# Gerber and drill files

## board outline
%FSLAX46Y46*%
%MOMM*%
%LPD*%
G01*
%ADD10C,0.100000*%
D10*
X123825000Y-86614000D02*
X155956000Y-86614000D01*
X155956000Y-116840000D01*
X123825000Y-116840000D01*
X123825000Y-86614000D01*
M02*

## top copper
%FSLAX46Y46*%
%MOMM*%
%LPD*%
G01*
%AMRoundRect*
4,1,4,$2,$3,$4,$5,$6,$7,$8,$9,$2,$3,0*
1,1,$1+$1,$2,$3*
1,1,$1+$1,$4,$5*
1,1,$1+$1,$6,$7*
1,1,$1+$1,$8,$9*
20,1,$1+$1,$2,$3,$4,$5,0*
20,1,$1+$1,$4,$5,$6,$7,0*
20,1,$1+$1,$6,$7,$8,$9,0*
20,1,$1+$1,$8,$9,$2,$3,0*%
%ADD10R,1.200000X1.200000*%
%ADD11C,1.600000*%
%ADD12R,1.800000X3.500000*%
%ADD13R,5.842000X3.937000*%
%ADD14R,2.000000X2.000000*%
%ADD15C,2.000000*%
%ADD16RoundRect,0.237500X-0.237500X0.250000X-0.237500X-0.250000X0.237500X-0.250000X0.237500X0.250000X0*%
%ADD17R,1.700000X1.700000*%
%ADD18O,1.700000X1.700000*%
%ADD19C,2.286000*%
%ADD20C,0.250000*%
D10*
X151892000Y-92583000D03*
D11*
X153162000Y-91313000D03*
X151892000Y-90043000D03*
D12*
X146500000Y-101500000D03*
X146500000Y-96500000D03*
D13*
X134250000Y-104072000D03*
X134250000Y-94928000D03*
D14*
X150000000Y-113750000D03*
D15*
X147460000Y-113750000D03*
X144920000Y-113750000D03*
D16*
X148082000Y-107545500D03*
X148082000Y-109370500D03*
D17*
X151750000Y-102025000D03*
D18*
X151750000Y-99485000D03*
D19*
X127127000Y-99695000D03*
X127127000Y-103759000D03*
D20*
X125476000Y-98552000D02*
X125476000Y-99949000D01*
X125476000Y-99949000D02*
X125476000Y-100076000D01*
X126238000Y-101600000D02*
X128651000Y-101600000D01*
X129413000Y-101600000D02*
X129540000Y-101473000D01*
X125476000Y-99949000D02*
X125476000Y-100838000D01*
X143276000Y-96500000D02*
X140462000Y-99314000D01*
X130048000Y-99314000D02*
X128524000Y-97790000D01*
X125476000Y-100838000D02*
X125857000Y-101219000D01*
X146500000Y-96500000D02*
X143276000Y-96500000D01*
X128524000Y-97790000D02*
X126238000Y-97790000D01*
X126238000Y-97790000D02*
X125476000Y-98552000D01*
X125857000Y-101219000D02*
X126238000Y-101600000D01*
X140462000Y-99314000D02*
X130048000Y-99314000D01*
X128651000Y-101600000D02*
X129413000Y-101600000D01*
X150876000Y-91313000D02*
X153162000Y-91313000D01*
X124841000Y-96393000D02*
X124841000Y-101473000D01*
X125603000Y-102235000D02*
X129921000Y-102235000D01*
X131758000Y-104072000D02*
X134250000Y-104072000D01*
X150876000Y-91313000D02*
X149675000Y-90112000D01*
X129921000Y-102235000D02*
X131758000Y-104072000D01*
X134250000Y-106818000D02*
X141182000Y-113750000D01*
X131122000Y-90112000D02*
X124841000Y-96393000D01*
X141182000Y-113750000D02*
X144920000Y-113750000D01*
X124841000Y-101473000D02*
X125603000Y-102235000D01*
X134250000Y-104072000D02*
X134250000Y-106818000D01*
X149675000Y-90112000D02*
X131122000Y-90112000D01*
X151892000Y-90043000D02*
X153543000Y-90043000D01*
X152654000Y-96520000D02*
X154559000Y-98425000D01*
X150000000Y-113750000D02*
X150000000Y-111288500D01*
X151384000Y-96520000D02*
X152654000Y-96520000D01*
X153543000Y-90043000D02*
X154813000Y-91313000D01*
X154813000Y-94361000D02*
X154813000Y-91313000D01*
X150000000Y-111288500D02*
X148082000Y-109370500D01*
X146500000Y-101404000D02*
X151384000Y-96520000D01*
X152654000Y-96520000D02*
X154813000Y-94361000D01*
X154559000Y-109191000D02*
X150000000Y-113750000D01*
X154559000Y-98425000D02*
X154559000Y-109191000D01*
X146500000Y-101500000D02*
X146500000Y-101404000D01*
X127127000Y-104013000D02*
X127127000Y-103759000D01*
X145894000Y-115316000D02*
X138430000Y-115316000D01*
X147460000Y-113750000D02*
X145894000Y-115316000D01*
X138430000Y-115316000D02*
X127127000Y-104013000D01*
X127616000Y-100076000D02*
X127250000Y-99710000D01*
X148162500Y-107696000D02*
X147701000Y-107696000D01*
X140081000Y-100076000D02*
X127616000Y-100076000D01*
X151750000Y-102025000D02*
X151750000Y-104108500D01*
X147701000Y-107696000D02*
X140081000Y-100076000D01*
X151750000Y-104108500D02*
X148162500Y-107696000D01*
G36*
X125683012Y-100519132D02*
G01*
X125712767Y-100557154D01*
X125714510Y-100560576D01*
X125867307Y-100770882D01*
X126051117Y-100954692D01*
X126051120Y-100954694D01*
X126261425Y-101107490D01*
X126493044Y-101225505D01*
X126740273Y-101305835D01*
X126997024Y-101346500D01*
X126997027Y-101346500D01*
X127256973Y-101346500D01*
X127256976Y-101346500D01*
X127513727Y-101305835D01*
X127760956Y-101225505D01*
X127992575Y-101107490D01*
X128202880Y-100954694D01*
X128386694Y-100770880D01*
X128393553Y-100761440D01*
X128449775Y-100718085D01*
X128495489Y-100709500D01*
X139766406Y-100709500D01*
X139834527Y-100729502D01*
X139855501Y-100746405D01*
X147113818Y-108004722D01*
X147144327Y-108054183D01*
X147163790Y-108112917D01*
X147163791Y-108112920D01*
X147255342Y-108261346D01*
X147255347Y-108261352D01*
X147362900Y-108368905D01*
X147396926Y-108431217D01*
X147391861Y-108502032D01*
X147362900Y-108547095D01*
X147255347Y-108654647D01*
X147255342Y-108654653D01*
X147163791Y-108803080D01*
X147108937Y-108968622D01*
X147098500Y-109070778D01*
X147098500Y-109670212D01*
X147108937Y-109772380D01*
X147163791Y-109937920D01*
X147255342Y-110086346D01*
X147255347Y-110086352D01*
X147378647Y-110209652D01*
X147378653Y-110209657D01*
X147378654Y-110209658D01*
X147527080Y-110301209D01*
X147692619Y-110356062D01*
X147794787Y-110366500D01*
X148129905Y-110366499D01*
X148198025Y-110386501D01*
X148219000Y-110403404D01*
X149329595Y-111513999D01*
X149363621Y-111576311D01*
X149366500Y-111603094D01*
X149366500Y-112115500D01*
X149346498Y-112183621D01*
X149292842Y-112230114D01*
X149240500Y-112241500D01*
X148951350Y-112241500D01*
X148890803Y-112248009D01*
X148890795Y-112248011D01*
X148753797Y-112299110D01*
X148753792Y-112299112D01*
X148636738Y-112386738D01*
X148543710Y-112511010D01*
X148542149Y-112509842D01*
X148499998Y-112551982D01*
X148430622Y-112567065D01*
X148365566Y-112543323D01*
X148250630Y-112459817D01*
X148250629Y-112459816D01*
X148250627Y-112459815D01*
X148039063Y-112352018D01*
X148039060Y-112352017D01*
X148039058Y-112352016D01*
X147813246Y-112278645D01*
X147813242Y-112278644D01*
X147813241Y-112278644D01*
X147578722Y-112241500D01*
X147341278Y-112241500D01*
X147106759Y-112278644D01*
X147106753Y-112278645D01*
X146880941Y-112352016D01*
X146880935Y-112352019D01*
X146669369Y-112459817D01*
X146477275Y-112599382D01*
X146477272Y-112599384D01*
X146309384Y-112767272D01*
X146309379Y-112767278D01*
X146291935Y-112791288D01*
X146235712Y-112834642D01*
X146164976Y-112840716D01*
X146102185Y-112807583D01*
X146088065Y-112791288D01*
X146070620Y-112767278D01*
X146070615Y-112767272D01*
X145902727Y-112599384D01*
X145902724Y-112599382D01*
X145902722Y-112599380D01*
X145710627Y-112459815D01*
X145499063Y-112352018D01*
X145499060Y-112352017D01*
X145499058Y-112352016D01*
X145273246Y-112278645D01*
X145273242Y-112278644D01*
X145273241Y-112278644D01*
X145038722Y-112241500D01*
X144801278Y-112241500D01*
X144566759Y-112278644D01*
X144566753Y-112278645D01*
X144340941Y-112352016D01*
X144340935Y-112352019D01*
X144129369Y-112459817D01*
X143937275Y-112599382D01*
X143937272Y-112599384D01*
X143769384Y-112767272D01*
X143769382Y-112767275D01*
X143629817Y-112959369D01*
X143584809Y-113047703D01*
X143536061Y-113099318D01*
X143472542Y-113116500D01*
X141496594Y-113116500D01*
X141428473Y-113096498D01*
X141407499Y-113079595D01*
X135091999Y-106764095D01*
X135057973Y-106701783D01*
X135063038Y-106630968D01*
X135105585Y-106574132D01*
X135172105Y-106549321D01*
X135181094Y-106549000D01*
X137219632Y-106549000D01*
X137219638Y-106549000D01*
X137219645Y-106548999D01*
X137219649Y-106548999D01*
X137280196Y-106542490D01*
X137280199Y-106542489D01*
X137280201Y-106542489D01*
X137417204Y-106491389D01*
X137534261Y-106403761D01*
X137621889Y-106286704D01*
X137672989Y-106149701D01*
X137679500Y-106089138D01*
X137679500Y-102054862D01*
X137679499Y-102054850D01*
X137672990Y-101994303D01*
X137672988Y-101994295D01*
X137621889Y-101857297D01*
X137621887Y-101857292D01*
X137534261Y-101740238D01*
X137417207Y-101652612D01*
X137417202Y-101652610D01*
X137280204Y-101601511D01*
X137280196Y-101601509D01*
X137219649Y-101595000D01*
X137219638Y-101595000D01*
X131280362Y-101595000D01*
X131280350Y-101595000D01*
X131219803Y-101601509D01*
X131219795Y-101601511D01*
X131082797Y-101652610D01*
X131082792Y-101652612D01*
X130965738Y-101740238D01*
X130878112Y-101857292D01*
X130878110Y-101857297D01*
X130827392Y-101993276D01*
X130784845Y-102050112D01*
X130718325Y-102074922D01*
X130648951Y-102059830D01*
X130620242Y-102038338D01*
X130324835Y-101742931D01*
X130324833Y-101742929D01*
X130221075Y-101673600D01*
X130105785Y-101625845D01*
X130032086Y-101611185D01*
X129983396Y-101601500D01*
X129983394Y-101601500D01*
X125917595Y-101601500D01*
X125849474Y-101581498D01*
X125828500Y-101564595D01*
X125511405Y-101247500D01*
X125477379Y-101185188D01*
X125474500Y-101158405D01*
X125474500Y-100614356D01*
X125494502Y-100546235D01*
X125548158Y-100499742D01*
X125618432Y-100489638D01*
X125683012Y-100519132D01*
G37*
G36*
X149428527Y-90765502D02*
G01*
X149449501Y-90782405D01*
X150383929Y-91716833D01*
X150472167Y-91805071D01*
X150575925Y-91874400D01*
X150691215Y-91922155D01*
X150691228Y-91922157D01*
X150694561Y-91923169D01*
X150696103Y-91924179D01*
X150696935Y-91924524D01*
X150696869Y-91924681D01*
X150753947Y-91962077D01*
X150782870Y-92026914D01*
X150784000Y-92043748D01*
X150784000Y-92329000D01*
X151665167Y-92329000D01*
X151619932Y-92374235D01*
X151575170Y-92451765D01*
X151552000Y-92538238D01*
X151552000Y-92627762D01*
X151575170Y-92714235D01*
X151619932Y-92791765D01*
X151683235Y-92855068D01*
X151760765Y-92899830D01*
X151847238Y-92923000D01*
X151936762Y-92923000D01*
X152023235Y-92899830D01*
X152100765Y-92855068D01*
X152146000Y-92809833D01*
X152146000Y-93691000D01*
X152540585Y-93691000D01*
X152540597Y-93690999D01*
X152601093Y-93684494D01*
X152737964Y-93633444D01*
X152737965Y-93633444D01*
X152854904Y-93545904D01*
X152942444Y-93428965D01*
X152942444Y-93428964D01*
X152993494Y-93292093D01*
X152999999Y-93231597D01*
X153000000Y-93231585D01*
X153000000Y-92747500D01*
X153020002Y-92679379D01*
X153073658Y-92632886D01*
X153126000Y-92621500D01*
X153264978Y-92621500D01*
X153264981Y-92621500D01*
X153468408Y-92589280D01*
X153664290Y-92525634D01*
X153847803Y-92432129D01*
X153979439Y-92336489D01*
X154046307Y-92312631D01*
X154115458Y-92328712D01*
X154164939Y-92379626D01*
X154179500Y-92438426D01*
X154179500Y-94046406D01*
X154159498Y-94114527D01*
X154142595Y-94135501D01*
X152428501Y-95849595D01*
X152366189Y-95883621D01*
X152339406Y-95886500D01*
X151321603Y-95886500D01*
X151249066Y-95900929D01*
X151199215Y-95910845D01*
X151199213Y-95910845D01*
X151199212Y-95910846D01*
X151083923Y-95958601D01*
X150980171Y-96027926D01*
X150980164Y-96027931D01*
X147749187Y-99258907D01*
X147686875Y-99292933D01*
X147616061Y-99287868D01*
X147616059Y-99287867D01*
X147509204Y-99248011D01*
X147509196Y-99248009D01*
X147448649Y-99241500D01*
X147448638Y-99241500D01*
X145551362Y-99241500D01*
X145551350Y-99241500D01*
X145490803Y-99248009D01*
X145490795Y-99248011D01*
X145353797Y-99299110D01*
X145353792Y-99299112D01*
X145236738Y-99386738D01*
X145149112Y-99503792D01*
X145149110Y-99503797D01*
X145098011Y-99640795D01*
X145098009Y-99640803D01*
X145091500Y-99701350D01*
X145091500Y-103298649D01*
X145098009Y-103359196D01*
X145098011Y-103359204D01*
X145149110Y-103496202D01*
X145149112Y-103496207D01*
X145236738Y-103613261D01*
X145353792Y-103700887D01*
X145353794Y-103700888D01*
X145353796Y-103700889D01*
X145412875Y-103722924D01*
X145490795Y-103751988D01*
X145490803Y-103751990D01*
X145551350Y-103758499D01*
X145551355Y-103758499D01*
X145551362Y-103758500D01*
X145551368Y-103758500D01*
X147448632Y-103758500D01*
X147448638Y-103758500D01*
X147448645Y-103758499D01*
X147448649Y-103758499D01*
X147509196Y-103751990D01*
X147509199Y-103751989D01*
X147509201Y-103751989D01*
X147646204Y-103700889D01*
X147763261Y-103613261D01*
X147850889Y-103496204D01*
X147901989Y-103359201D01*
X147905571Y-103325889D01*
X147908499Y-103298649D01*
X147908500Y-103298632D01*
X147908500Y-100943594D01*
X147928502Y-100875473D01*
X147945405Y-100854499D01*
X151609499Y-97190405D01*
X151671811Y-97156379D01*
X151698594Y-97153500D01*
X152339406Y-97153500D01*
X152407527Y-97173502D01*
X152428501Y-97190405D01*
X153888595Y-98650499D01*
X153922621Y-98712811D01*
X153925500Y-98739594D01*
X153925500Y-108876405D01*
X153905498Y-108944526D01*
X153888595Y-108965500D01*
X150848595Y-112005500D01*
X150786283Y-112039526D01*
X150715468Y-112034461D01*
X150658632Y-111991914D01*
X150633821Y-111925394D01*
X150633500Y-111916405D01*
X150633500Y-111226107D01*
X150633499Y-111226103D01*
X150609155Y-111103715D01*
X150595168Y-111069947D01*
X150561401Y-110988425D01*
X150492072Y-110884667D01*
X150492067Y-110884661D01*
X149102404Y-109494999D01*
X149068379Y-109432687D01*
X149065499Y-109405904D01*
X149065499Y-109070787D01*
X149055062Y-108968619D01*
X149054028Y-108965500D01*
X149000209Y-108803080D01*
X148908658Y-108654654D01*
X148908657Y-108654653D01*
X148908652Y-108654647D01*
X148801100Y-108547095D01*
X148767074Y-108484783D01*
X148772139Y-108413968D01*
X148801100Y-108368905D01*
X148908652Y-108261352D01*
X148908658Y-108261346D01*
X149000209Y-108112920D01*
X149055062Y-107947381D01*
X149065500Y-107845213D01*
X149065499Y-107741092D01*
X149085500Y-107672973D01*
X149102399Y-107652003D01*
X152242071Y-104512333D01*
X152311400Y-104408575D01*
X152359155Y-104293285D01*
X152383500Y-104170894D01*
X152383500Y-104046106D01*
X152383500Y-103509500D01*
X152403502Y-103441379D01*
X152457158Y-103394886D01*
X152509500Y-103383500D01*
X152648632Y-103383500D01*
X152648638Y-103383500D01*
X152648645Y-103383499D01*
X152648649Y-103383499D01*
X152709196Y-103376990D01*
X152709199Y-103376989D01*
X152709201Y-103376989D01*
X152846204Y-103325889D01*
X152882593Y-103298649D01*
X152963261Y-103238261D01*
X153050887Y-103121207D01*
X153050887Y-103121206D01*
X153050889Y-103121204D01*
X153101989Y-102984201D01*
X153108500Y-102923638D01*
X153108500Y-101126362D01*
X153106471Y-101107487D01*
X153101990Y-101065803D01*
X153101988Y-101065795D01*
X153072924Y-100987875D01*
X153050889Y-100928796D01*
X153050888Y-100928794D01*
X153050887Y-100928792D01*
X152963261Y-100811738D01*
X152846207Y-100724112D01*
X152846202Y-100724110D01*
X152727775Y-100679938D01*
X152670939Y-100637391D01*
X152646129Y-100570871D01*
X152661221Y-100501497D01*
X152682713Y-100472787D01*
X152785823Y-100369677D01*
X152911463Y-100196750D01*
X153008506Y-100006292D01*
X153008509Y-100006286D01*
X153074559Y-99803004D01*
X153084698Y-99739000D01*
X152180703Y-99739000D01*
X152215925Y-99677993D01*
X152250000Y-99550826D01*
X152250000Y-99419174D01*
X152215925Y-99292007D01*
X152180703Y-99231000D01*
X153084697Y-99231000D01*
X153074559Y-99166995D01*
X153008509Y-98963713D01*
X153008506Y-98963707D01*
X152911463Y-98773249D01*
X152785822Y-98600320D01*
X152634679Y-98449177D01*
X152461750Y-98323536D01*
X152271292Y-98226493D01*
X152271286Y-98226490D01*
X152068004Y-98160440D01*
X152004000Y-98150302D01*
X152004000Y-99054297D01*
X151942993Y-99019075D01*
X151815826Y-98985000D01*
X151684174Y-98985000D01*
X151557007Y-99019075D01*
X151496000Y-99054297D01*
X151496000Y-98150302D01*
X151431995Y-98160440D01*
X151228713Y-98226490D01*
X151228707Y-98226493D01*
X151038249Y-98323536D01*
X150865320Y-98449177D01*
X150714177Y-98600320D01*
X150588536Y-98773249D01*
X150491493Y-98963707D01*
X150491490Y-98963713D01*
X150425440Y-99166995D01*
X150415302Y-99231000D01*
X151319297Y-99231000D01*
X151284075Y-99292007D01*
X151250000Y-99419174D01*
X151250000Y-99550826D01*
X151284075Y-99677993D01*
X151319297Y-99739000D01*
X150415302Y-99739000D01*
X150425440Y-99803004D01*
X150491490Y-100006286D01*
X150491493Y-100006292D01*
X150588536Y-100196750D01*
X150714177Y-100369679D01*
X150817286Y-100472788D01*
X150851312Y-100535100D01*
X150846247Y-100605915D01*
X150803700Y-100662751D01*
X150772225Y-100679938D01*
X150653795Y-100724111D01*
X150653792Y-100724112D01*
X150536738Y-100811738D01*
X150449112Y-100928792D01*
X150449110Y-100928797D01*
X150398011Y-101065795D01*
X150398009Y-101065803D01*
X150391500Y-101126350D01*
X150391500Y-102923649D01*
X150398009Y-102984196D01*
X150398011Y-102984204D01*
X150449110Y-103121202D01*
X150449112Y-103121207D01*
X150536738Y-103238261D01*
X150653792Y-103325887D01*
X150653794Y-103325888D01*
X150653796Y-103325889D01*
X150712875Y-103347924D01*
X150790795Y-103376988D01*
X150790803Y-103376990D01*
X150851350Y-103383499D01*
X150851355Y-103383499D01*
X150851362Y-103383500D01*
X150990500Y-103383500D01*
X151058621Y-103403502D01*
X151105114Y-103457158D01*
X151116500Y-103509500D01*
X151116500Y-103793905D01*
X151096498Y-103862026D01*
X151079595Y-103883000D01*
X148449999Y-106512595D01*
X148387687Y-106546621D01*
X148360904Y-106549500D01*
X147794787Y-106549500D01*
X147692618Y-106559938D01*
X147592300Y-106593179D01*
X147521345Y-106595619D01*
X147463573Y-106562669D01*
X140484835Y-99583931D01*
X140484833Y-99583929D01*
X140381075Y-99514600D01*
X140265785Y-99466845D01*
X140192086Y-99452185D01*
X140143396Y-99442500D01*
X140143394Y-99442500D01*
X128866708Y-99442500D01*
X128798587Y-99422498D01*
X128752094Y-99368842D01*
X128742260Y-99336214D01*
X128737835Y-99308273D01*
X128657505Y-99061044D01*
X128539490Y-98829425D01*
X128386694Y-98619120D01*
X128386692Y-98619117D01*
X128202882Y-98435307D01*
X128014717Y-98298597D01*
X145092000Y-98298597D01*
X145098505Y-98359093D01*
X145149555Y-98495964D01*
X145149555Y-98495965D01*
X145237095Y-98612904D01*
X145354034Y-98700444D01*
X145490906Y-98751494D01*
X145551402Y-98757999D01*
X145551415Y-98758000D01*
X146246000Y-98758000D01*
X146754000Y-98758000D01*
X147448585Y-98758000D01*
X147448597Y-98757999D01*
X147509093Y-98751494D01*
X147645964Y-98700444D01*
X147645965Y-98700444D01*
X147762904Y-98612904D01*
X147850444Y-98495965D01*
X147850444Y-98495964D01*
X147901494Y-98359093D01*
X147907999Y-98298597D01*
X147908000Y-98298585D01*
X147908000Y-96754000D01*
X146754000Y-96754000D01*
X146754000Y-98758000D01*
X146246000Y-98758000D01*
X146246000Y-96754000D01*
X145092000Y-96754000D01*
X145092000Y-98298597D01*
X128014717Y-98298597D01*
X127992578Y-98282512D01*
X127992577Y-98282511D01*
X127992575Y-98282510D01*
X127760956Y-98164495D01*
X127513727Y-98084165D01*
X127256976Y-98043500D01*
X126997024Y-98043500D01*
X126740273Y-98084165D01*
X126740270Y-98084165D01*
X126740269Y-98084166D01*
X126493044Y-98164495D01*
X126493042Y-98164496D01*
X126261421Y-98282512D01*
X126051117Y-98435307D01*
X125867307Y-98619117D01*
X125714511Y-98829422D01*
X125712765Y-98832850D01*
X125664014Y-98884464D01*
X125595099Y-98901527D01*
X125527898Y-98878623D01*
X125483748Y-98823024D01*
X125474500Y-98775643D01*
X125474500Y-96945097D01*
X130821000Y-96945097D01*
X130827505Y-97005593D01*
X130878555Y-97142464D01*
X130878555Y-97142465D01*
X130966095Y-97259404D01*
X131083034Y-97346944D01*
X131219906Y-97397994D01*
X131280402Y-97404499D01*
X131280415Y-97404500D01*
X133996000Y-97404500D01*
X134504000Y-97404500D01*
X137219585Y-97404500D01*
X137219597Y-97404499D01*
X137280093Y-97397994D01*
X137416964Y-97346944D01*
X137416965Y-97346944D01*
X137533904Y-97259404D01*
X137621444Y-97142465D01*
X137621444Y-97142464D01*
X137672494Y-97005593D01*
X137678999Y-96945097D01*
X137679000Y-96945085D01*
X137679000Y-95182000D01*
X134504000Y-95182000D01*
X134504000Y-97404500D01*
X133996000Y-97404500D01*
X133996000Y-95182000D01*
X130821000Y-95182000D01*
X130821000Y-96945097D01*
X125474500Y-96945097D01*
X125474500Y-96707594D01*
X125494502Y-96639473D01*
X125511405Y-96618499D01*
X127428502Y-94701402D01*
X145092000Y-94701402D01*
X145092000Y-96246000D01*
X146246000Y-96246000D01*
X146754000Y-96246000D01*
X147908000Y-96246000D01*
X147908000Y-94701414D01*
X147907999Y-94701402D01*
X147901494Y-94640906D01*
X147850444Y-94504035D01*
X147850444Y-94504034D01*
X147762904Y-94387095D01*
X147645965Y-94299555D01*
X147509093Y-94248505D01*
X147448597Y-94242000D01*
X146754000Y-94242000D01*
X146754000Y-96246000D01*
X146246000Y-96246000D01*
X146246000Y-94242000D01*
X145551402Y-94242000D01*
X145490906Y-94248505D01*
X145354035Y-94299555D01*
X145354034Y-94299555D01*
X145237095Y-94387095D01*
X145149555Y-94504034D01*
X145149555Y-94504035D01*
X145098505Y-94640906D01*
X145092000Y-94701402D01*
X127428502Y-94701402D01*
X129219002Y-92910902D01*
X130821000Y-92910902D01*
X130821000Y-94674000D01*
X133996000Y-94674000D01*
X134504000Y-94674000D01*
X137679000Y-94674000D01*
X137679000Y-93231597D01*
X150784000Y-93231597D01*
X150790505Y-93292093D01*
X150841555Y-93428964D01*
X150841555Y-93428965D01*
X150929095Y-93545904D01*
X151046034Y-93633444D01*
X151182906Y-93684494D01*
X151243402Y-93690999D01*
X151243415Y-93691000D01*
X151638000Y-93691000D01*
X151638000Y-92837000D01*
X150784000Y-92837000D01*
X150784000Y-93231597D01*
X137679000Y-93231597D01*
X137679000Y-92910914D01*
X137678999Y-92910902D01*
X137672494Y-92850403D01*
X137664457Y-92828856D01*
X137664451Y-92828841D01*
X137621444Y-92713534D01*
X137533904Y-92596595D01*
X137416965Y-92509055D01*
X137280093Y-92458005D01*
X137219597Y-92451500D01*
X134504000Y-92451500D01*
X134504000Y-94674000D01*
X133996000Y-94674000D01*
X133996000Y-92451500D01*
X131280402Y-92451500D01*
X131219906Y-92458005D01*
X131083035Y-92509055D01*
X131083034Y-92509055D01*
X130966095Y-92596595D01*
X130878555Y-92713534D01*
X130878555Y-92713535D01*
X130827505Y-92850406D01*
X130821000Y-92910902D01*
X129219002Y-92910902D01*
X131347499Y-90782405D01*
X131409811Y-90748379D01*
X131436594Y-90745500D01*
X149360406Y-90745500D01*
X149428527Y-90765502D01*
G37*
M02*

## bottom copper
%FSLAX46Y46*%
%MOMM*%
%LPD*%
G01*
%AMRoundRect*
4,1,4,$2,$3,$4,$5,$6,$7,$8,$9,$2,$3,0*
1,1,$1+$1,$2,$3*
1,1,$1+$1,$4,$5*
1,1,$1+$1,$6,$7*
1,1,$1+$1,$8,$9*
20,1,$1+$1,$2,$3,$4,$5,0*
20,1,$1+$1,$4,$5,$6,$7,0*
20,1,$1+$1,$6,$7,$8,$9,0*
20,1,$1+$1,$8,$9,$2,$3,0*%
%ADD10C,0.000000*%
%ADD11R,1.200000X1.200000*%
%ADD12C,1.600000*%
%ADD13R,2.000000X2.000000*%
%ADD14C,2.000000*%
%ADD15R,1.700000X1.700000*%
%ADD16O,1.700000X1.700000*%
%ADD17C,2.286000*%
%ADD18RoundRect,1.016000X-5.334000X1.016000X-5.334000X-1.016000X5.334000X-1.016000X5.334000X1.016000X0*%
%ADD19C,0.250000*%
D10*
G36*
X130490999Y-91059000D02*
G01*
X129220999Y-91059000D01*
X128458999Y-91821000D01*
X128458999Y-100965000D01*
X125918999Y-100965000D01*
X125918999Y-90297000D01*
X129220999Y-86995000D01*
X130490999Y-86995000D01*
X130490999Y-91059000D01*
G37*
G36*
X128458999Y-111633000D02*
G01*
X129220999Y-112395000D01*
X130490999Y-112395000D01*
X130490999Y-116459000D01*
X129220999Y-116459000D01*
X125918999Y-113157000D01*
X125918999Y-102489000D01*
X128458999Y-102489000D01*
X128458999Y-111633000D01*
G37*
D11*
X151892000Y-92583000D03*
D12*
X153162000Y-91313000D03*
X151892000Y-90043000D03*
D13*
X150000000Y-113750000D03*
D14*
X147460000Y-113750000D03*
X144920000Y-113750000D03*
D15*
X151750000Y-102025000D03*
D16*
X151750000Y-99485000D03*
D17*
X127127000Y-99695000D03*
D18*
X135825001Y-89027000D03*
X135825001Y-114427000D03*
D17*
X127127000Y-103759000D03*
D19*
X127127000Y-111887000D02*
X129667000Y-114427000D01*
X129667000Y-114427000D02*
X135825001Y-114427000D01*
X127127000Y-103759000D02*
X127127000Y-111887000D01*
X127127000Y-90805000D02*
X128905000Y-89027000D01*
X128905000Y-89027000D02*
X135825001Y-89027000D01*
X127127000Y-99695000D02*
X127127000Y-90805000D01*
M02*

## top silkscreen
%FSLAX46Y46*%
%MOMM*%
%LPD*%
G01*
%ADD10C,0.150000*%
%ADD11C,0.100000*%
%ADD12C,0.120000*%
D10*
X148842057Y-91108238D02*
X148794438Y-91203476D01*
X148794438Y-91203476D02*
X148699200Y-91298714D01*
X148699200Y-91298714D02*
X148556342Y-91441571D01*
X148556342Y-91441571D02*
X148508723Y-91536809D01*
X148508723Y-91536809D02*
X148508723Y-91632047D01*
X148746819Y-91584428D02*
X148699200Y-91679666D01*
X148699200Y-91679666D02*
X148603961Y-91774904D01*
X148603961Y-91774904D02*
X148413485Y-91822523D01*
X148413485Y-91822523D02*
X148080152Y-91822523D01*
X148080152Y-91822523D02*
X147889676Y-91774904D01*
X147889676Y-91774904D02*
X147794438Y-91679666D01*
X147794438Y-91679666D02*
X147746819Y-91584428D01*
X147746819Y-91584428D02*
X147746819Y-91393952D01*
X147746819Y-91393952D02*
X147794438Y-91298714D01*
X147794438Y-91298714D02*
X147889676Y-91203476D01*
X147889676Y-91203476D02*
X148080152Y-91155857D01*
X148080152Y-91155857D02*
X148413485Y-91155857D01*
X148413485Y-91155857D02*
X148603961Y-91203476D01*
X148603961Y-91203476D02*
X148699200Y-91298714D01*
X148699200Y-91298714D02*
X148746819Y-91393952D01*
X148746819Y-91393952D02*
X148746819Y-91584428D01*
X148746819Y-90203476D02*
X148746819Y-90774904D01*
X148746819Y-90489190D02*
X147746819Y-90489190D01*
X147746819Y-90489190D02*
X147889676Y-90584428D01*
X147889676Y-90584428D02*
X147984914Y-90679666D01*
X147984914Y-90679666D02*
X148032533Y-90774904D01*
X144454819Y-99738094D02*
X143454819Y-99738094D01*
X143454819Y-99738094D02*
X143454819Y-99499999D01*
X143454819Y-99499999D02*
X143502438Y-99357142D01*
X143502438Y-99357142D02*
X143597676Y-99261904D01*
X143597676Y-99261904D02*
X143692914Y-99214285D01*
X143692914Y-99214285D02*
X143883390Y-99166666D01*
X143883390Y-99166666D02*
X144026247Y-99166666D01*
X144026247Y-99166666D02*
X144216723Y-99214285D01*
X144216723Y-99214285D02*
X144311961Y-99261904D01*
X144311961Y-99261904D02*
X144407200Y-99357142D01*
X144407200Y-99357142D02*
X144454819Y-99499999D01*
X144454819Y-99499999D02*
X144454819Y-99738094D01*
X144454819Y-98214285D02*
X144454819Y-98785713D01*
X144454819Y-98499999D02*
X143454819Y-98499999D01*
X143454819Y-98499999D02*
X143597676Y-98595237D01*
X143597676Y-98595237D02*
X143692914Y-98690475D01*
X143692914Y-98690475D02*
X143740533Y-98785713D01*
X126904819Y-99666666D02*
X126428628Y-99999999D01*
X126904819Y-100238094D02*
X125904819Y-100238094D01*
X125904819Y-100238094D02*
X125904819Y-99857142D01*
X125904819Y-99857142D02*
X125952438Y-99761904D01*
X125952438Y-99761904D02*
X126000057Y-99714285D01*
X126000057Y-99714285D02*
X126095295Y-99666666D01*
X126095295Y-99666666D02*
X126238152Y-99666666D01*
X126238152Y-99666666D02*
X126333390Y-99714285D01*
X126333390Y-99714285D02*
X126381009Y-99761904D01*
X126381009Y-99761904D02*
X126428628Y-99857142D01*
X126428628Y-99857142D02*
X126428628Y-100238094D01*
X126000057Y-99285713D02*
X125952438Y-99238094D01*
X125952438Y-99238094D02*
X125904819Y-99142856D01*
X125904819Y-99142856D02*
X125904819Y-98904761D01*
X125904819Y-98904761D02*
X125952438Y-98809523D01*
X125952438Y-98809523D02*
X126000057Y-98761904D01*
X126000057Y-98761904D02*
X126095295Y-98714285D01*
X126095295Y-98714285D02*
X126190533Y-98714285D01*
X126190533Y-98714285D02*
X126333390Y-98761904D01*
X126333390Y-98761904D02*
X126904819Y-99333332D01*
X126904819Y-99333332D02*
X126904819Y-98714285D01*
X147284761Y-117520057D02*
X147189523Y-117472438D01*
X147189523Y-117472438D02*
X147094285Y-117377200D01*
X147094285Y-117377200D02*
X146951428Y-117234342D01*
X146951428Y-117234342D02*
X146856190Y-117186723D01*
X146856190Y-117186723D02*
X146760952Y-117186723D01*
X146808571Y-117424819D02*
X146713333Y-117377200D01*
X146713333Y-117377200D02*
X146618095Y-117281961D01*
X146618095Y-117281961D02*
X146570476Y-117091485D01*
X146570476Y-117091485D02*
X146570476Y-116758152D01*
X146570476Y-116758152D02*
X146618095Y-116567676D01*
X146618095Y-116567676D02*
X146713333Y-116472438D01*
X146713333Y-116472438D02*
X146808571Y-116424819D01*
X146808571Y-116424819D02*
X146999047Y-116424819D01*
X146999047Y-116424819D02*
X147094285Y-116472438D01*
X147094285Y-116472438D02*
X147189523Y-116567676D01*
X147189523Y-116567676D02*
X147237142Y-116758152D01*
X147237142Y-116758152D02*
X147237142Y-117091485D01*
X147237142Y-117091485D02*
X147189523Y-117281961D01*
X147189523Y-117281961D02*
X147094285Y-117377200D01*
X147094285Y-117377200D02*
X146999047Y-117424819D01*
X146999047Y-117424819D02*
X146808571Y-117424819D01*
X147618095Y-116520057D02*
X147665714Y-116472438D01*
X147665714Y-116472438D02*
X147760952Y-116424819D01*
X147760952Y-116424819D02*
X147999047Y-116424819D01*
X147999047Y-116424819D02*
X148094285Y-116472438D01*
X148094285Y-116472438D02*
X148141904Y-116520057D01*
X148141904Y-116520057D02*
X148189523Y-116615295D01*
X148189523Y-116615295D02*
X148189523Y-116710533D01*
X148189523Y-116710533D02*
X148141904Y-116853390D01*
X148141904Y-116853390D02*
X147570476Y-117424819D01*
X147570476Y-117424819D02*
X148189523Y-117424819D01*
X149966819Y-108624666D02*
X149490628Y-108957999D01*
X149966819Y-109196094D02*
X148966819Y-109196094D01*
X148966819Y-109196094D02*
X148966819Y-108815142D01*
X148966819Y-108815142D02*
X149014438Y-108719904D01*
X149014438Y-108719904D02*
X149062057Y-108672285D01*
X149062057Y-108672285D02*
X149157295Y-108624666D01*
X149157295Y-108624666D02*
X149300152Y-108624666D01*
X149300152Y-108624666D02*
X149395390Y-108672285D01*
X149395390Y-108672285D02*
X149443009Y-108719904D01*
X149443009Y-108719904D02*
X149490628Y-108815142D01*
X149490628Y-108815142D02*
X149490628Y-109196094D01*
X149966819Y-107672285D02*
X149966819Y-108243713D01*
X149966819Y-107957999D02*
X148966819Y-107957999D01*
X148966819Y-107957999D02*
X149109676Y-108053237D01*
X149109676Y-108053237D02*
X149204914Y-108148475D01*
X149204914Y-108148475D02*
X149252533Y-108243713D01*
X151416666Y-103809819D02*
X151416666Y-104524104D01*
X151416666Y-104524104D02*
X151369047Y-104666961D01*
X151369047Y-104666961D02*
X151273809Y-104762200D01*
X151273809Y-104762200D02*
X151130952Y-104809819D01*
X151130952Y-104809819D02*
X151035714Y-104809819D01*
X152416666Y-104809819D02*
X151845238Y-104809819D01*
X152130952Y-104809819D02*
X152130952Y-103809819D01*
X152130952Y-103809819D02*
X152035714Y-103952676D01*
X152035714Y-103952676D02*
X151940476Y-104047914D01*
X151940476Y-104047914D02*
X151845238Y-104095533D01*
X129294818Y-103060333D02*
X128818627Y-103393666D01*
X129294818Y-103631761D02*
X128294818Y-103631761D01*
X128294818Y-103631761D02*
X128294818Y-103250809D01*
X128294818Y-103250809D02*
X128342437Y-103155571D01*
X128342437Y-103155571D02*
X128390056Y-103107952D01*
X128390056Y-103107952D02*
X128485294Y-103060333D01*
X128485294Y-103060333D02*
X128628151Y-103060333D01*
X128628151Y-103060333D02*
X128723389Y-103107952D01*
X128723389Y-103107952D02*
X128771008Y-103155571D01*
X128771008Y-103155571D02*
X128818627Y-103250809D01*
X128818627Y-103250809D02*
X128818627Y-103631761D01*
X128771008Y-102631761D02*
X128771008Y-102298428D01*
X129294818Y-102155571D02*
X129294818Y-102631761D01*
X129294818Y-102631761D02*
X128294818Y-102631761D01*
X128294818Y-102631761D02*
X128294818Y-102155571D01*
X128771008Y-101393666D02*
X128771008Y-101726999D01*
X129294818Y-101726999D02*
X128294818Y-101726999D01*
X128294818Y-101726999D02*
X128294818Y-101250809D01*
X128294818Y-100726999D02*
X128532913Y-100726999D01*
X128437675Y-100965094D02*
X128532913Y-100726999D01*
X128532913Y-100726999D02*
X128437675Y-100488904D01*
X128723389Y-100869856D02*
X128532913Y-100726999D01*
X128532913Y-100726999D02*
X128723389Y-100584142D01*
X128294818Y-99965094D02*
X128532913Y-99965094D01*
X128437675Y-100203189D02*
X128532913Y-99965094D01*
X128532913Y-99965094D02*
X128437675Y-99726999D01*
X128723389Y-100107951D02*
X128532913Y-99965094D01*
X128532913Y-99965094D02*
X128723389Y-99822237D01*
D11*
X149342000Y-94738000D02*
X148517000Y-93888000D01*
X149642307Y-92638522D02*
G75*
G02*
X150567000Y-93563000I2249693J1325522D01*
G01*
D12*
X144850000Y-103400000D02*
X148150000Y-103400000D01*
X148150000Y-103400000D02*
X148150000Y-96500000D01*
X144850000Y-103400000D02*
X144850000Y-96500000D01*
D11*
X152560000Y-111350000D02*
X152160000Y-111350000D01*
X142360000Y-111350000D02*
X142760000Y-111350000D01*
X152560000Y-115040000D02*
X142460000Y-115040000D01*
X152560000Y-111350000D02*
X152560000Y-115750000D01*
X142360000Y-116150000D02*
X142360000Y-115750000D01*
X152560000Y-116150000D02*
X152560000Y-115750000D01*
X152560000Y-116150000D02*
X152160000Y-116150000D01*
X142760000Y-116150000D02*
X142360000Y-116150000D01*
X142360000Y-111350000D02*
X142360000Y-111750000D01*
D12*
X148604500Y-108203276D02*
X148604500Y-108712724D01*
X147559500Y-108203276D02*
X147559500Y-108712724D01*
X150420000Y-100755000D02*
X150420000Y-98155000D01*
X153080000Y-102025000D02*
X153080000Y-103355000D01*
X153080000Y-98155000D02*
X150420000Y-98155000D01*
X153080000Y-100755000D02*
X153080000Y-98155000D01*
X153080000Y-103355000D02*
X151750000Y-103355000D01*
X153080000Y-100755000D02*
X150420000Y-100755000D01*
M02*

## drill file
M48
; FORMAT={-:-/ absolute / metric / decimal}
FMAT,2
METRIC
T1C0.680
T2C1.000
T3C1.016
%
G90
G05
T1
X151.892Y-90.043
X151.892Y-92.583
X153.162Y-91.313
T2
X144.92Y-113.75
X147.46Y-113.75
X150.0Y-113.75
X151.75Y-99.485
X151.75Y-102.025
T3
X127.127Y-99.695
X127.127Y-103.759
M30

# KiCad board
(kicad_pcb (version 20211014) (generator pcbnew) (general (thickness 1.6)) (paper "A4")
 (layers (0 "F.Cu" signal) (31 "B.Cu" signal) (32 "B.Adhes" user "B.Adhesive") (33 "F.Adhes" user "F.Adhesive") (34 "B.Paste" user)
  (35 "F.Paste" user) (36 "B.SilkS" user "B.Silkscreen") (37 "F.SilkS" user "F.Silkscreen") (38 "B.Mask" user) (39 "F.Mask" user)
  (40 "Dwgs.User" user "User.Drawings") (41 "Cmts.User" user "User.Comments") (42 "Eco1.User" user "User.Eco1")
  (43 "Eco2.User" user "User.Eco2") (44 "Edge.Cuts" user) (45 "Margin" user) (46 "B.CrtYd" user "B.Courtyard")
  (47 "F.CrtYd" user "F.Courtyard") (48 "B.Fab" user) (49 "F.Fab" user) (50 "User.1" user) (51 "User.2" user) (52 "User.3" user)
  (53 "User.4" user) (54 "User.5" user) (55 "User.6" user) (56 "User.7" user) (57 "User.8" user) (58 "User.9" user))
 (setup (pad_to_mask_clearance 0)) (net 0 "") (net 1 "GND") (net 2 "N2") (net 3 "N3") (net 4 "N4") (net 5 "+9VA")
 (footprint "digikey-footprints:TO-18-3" (layer "F.Cu") (at 151.892 92.583 90)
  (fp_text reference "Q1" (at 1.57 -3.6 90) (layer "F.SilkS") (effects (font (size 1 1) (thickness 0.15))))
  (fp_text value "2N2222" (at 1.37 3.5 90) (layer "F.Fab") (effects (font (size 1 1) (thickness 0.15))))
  (fp_line (start -2.155 -2.55) (end -1.305 -3.375) (layer "F.SilkS") (width 0.1))
  (fp_arc (start -0.055522 -2.249693) (mid 3.116581 1.846151) (end -0.98 -1.325) (layer "F.SilkS") (width 0.1))
  (pad "1" thru_hole rect locked (at 0 0 90) (size 1.2 1.2) (drill 0.68) (layers *.Cu *.Mask) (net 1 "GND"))
  (pad "2" thru_hole circle locked (at 1.27 1.27 90) (size 1.6 1.6) (drill 0.68) (layers *.Cu *.Mask) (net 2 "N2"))
  (pad "3" thru_hole circle locked (at 2.54 0 90) (size 1.6 1.6) (drill 0.68) (layers *.Cu *.Mask) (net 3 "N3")))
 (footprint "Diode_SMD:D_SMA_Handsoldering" (layer "F.Cu") (at 146.5 99 90)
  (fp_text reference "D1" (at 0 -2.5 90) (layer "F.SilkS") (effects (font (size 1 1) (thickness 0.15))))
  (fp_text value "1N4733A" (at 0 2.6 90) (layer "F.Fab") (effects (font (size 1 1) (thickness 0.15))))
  (fp_line (start -4.4 -1.65) (end -4.4 1.65) (layer "F.SilkS") (width 0.12))
  (fp_line (start -4.4 1.65) (end 2.5 1.65) (layer "F.SilkS") (width 0.12))
  (fp_line (start -4.4 -1.65) (end 2.5 -1.65) (layer "F.SilkS") (width 0.12))
  (pad "1" smd rect locked (at -2.5 0 90) (size 3.5 1.8) (layers "F.Cu" "F.Paste" "F.Mask") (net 3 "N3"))
  (pad "2" smd rect locked (at 2.5 0 90) (size 3.5 1.8) (layers "F.Cu" "F.Paste" "F.Mask") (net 1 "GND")))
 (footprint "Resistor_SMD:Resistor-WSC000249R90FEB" (layer "F.Cu") (at 134.25 99.5 90)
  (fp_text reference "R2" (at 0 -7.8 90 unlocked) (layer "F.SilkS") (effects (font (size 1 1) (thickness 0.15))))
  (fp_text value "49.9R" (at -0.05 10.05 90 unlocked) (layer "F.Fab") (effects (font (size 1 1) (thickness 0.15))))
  (pad "1" smd rect (at -4.572 0 90) (size 3.937 5.842) (layers "F.Cu" "F.Paste" "F.Mask") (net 2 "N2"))
  (pad "2" smd rect (at 4.572 0 90) (size 3.937 5.842) (layers "F.Cu" "F.Paste" "F.Mask") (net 1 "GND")))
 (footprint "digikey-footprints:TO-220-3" (layer "F.Cu") (at 150 113.75 180)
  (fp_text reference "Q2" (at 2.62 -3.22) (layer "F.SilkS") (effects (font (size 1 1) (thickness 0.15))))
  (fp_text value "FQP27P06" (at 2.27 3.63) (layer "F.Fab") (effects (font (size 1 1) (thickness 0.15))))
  (fp_line (start -2.56 2.4) (end -2.16 2.4) (layer "F.SilkS") (width 0.1))
  (fp_line (start 7.64 2.4) (end 7.24 2.4) (layer "F.SilkS") (width 0.1))
  (fp_line (start -2.56 -1.29) (end 7.54 -1.29) (layer "F.SilkS") (width 0.1))
  (fp_line (start -2.56 2.4) (end -2.56 -2) (layer "F.SilkS") (width 0.1))
  (fp_line (start 7.64 -2.4) (end 7.64 -2) (layer "F.SilkS") (width 0.1))
  (fp_line (start -2.56 -2.4) (end -2.56 -2) (layer "F.SilkS") (width 0.1))
  (fp_line (start -2.56 -2.4) (end -2.16 -2.4) (layer "F.SilkS") (width 0.1))
  (fp_line (start 7.24 -2.4) (end 7.64 -2.4) (layer "F.SilkS") (width 0.1))
  (fp_line (start 7.64 2.4) (end 7.64 2) (layer "F.SilkS") (width 0.1))
  (pad "1" thru_hole rect locked (at 0 0 180) (size 2 2) (drill 1) (layers *.Cu *.Mask) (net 3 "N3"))
  (pad "2" thru_hole circle locked (at 2.54 0 180) (size 2 2) (drill 1) (layers *.Cu *.Mask) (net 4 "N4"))
  (pad "3" thru_hole circle locked (at 5.08 0 180) (size 2 2) (drill 1) (layers *.Cu *.Mask) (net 2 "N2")))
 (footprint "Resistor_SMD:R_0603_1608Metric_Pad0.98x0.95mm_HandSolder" (layer "F.Cu") (at 148.082 108.458 -90)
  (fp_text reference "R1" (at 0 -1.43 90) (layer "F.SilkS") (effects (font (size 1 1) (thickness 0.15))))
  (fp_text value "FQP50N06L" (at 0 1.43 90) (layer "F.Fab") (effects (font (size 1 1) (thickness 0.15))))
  (fp_line (start -0.254724 -0.5225) (end 0.254724 -0.5225) (layer "F.SilkS") (width 0.12))
  (fp_line (start -0.254724 0.5225) (end 0.254724 0.5225) (layer "F.SilkS") (width 0.12))
  (pad "1" smd roundrect locked (at -0.9125 0 270) (size 0.975 0.95) (layers "F.Cu" "F.Paste" "F.Mask") (roundrect_rratio 0.25)
   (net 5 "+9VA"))
  (pad "2" smd roundrect locked (at 0.9125 0 270) (size 0.975 0.95) (layers "F.Cu" "F.Paste" "F.Mask") (roundrect_rratio 0.25) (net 3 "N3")))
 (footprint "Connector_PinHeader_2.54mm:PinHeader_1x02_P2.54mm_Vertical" (layer "F.Cu") (at 151.75 102.025 180)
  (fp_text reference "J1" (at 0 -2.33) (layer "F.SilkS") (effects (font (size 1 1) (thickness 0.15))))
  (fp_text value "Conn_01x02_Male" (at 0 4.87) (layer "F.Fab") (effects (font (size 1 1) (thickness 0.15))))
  (fp_line (start 1.33 1.27) (end 1.33 3.87) (layer "F.SilkS") (width 0.12))
  (fp_line (start -1.33 0) (end -1.33 -1.33) (layer "F.SilkS") (width 0.12))
  (fp_line (start -1.33 3.87) (end 1.33 3.87) (layer "F.SilkS") (width 0.12))
  (fp_line (start -1.33 1.27) (end -1.33 3.87) (layer "F.SilkS") (width 0.12))
  (fp_line (start -1.33 -1.33) (end 0 -1.33) (layer "F.SilkS") (width 0.12))
  (fp_line (start -1.33 1.27) (end 1.33 1.27) (layer "F.SilkS") (width 0.12))
  (pad "1" thru_hole rect locked (at 0 0 180) (size 1.7 1.7) (drill 1) (layers *.Cu *.Mask) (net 5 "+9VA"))
  (pad "2" thru_hole oval locked (at 0 2.54 180) (size 1.7 1.7) (drill 1) (layers *.Cu *.Mask) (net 1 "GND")))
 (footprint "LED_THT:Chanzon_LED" (layer "F.Cu") (at 139.126999 101.727 90)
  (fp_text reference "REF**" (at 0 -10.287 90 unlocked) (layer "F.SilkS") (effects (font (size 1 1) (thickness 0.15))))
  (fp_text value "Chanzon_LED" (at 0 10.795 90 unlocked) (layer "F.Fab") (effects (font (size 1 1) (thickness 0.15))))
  (fp_poly
   (pts (xy 0.762 -10.668) (xy 9.906 -10.668) (xy 10.668 -9.906) (xy 10.668 -8.636) (xy 14.732 -8.636) (xy 14.732 -9.906) (xy 11.43 -13.208)
    (xy 0.762 -13.208))
   (layer "B.Cu") (width 0) (fill solid))
  (fp_poly
   (pts (xy -0.762 -10.668) (xy -9.906 -10.668) (xy -10.668 -9.906) (xy -10.668 -8.636) (xy -14.732 -8.636) (xy -14.732 -9.906)
    (xy -11.43 -13.208) (xy -0.762 -13.208))
   (layer "B.Cu") (width 0) (fill solid))
  (pad "1" thru_hole circle (at 2.032 -11.999999) (size 2.286 2.286) (drill 1.016) (layers *.Cu *.Mask) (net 5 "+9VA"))
  (pad "1" smd roundrect (at 12.7 -3.301998 270) (size 4.064 12.7) (layers "B.Cu" "B.Paste" "B.Mask") (roundrect_rratio 0.25) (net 5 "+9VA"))
  (pad "2" smd roundrect (at -12.7 -3.301998 270) (size 4.064 12.7) (layers "B.Cu" "B.Paste" "B.Mask") (roundrect_rratio 0.25) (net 4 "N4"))
  (pad "2" thru_hole circle (at -2.032 -11.999999) (size 2.286 2.286) (drill 1.016) (layers *.Cu *.Mask) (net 4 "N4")))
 (gr_rect (start 123.825 86.614) (end 155.956 116.84) (layer "Edge.Cuts") (width 0.1) (fill none))
 (segment (start 125.476 98.552) (end 125.476 99.949) (width 0.25) (layer "F.Cu") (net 1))
 (segment (start 125.476 99.949) (end 125.476 100.076) (width 0.25) (layer "F.Cu") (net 1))
 (segment (start 126.238 101.6) (end 128.651 101.6) (width 0.25) (layer "F.Cu") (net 1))
 (segment (start 129.413 101.6) (end 129.54 101.473) (width 0.25) (layer "F.Cu") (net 1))
 (segment (start 125.476 99.949) (end 125.476 100.838) (width 0.25) (layer "F.Cu") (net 1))
 (segment (start 143.276 96.5) (end 140.462 99.314) (width 0.25) (layer "F.Cu") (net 1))
 (segment (start 130.048 99.314) (end 128.524 97.79) (width 0.25) (layer "F.Cu") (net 1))
 (segment (start 125.476 100.838) (end 125.857 101.219) (width 0.25) (layer "F.Cu") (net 1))
 (segment (start 146.5 96.5) (end 143.276 96.5) (width 0.25) (layer "F.Cu") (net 1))
 (segment (start 128.524 97.79) (end 126.238 97.79) (width 0.25) (layer "F.Cu") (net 1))
 (segment (start 126.238 97.79) (end 125.476 98.552) (width 0.25) (layer "F.Cu") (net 1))
 (segment (start 125.857 101.219) (end 126.238 101.6) (width 0.25) (layer "F.Cu") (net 1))
 (segment (start 140.462 99.314) (end 130.048 99.314) (width 0.25) (layer "F.Cu") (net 1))
 (segment (start 128.651 101.6) (end 129.413 101.6) (width 0.25) (layer "F.Cu") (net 1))
 (segment (start 150.876 91.313) (end 153.162 91.313) (width 0.25) (layer "F.Cu") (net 2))
 (segment (start 124.841 96.393) (end 124.841 101.473) (width 0.25) (layer "F.Cu") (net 2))
 (segment (start 125.603 102.235) (end 129.921 102.235) (width 0.25) (layer "F.Cu") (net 2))
 (segment (start 131.758 104.072) (end 134.25 104.072) (width 0.25) (layer "F.Cu") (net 2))
 (segment (start 150.876 91.313) (end 149.675 90.112) (width 0.25) (layer "F.Cu") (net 2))
 (segment (start 129.921 102.235) (end 131.758 104.072) (width 0.25) (layer "F.Cu") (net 2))
 (segment (start 134.25 106.818) (end 141.182 113.75) (width 0.25) (layer "F.Cu") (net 2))
 (segment (start 131.122 90.112) (end 124.841 96.393) (width 0.25) (layer "F.Cu") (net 2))
 (segment (start 141.182 113.75) (end 144.92 113.75) (width 0.25) (layer "F.Cu") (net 2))
 (segment (start 124.841 101.473) (end 125.603 102.235) (width 0.25) (layer "F.Cu") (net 2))
 (segment (start 134.25 104.072) (end 134.25 106.818) (width 0.25) (layer "F.Cu") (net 2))
 (segment (start 149.675 90.112) (end 131.122 90.112) (width 0.25) (layer "F.Cu") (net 2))
 (segment (start 151.892 90.043) (end 153.543 90.043) (width 0.25) (layer "F.Cu") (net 3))
 (segment (start 152.654 96.52) (end 154.559 98.425) (width 0.25) (layer "F.Cu") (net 3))
 (segment (start 150 113.75) (end 150 111.2885) (width 0.25) (layer "F.Cu") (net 3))
 (segment (start 151.384 96.52) (end 152.654 96.52) (width 0.25) (layer "F.Cu") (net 3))
 (segment (start 153.543 90.043) (end 154.813 91.313) (width 0.25) (layer "F.Cu") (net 3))
 (segment (start 154.813 94.361) (end 154.813 91.313) (width 0.25) (layer "F.Cu") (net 3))
 (segment (start 150 111.2885) (end 148.082 109.3705) (width 0.25) (layer "F.Cu") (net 3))
 (segment (start 146.5 101.404) (end 151.384 96.52) (width 0.25) (layer "F.Cu") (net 3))
 (segment (start 152.654 96.52) (end 154.813 94.361) (width 0.25) (layer "F.Cu") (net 3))
 (segment (start 154.559 109.191) (end 150 113.75) (width 0.25) (layer "F.Cu") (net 3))
 (segment (start 154.559 98.425) (end 154.559 109.191) (width 0.25) (layer "F.Cu") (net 3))
 (segment (start 146.5 101.5) (end 146.5 101.404) (width 0.25) (layer "F.Cu") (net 3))
 (segment (start 127.127 104.013) (end 127.127 103.759) (width 0.25) (layer "F.Cu") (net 4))
 (segment (start 145.894 115.316) (end 138.43 115.316) (width 0.25) (layer "F.Cu") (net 4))
 (segment (start 147.46 113.75) (end 145.894 115.316) (width 0.25) (layer "F.Cu") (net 4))
 (segment (start 138.43 115.316) (end 127.127 104.013) (width 0.25) (layer "F.Cu") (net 4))
 (segment (start 127.127 111.887) (end 129.667 114.427) (width 0.25) (layer "B.Cu") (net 4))
 (segment (start 129.667 114.427) (end 135.825001 114.427) (width 0.25) (layer "B.Cu") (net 4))
 (segment (start 127.127 103.759) (end 127.127 111.887) (width 0.25) (layer "B.Cu") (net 4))
 (segment (start 127.616 100.076) (end 127.25 99.71) (width 0.25) (layer "F.Cu") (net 5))
 (segment (start 148.1625 107.696) (end 147.701 107.696) (width 0.25) (layer "F.Cu") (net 5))
 (segment (start 140.081 100.076) (end 127.616 100.076) (width 0.25) (layer "F.Cu") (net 5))
 (segment (start 151.75 102.025) (end 151.75 104.1085) (width 0.25) (layer "F.Cu") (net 5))
 (segment (start 147.701 107.696) (end 140.081 100.076) (width 0.25) (layer "F.Cu") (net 5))
 (segment (start 151.75 104.1085) (end 148.1625 107.696) (width 0.25) (layer "F.Cu") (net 5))
 (segment (start 127.127 90.805) (end 128.905 89.027) (width 0.25) (layer "B.Cu") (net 5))
 (segment (start 128.905 89.027) (end 135.825001 89.027) (width 0.25) (layer "B.Cu") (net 5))
 (segment (start 127.127 99.695) (end 127.127 90.805) (width 0.25) (layer "B.Cu") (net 5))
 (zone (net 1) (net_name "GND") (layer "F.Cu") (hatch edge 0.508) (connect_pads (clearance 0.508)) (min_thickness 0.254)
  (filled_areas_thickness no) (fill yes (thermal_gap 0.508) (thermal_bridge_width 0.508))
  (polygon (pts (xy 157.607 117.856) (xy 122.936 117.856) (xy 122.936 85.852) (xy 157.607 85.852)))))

